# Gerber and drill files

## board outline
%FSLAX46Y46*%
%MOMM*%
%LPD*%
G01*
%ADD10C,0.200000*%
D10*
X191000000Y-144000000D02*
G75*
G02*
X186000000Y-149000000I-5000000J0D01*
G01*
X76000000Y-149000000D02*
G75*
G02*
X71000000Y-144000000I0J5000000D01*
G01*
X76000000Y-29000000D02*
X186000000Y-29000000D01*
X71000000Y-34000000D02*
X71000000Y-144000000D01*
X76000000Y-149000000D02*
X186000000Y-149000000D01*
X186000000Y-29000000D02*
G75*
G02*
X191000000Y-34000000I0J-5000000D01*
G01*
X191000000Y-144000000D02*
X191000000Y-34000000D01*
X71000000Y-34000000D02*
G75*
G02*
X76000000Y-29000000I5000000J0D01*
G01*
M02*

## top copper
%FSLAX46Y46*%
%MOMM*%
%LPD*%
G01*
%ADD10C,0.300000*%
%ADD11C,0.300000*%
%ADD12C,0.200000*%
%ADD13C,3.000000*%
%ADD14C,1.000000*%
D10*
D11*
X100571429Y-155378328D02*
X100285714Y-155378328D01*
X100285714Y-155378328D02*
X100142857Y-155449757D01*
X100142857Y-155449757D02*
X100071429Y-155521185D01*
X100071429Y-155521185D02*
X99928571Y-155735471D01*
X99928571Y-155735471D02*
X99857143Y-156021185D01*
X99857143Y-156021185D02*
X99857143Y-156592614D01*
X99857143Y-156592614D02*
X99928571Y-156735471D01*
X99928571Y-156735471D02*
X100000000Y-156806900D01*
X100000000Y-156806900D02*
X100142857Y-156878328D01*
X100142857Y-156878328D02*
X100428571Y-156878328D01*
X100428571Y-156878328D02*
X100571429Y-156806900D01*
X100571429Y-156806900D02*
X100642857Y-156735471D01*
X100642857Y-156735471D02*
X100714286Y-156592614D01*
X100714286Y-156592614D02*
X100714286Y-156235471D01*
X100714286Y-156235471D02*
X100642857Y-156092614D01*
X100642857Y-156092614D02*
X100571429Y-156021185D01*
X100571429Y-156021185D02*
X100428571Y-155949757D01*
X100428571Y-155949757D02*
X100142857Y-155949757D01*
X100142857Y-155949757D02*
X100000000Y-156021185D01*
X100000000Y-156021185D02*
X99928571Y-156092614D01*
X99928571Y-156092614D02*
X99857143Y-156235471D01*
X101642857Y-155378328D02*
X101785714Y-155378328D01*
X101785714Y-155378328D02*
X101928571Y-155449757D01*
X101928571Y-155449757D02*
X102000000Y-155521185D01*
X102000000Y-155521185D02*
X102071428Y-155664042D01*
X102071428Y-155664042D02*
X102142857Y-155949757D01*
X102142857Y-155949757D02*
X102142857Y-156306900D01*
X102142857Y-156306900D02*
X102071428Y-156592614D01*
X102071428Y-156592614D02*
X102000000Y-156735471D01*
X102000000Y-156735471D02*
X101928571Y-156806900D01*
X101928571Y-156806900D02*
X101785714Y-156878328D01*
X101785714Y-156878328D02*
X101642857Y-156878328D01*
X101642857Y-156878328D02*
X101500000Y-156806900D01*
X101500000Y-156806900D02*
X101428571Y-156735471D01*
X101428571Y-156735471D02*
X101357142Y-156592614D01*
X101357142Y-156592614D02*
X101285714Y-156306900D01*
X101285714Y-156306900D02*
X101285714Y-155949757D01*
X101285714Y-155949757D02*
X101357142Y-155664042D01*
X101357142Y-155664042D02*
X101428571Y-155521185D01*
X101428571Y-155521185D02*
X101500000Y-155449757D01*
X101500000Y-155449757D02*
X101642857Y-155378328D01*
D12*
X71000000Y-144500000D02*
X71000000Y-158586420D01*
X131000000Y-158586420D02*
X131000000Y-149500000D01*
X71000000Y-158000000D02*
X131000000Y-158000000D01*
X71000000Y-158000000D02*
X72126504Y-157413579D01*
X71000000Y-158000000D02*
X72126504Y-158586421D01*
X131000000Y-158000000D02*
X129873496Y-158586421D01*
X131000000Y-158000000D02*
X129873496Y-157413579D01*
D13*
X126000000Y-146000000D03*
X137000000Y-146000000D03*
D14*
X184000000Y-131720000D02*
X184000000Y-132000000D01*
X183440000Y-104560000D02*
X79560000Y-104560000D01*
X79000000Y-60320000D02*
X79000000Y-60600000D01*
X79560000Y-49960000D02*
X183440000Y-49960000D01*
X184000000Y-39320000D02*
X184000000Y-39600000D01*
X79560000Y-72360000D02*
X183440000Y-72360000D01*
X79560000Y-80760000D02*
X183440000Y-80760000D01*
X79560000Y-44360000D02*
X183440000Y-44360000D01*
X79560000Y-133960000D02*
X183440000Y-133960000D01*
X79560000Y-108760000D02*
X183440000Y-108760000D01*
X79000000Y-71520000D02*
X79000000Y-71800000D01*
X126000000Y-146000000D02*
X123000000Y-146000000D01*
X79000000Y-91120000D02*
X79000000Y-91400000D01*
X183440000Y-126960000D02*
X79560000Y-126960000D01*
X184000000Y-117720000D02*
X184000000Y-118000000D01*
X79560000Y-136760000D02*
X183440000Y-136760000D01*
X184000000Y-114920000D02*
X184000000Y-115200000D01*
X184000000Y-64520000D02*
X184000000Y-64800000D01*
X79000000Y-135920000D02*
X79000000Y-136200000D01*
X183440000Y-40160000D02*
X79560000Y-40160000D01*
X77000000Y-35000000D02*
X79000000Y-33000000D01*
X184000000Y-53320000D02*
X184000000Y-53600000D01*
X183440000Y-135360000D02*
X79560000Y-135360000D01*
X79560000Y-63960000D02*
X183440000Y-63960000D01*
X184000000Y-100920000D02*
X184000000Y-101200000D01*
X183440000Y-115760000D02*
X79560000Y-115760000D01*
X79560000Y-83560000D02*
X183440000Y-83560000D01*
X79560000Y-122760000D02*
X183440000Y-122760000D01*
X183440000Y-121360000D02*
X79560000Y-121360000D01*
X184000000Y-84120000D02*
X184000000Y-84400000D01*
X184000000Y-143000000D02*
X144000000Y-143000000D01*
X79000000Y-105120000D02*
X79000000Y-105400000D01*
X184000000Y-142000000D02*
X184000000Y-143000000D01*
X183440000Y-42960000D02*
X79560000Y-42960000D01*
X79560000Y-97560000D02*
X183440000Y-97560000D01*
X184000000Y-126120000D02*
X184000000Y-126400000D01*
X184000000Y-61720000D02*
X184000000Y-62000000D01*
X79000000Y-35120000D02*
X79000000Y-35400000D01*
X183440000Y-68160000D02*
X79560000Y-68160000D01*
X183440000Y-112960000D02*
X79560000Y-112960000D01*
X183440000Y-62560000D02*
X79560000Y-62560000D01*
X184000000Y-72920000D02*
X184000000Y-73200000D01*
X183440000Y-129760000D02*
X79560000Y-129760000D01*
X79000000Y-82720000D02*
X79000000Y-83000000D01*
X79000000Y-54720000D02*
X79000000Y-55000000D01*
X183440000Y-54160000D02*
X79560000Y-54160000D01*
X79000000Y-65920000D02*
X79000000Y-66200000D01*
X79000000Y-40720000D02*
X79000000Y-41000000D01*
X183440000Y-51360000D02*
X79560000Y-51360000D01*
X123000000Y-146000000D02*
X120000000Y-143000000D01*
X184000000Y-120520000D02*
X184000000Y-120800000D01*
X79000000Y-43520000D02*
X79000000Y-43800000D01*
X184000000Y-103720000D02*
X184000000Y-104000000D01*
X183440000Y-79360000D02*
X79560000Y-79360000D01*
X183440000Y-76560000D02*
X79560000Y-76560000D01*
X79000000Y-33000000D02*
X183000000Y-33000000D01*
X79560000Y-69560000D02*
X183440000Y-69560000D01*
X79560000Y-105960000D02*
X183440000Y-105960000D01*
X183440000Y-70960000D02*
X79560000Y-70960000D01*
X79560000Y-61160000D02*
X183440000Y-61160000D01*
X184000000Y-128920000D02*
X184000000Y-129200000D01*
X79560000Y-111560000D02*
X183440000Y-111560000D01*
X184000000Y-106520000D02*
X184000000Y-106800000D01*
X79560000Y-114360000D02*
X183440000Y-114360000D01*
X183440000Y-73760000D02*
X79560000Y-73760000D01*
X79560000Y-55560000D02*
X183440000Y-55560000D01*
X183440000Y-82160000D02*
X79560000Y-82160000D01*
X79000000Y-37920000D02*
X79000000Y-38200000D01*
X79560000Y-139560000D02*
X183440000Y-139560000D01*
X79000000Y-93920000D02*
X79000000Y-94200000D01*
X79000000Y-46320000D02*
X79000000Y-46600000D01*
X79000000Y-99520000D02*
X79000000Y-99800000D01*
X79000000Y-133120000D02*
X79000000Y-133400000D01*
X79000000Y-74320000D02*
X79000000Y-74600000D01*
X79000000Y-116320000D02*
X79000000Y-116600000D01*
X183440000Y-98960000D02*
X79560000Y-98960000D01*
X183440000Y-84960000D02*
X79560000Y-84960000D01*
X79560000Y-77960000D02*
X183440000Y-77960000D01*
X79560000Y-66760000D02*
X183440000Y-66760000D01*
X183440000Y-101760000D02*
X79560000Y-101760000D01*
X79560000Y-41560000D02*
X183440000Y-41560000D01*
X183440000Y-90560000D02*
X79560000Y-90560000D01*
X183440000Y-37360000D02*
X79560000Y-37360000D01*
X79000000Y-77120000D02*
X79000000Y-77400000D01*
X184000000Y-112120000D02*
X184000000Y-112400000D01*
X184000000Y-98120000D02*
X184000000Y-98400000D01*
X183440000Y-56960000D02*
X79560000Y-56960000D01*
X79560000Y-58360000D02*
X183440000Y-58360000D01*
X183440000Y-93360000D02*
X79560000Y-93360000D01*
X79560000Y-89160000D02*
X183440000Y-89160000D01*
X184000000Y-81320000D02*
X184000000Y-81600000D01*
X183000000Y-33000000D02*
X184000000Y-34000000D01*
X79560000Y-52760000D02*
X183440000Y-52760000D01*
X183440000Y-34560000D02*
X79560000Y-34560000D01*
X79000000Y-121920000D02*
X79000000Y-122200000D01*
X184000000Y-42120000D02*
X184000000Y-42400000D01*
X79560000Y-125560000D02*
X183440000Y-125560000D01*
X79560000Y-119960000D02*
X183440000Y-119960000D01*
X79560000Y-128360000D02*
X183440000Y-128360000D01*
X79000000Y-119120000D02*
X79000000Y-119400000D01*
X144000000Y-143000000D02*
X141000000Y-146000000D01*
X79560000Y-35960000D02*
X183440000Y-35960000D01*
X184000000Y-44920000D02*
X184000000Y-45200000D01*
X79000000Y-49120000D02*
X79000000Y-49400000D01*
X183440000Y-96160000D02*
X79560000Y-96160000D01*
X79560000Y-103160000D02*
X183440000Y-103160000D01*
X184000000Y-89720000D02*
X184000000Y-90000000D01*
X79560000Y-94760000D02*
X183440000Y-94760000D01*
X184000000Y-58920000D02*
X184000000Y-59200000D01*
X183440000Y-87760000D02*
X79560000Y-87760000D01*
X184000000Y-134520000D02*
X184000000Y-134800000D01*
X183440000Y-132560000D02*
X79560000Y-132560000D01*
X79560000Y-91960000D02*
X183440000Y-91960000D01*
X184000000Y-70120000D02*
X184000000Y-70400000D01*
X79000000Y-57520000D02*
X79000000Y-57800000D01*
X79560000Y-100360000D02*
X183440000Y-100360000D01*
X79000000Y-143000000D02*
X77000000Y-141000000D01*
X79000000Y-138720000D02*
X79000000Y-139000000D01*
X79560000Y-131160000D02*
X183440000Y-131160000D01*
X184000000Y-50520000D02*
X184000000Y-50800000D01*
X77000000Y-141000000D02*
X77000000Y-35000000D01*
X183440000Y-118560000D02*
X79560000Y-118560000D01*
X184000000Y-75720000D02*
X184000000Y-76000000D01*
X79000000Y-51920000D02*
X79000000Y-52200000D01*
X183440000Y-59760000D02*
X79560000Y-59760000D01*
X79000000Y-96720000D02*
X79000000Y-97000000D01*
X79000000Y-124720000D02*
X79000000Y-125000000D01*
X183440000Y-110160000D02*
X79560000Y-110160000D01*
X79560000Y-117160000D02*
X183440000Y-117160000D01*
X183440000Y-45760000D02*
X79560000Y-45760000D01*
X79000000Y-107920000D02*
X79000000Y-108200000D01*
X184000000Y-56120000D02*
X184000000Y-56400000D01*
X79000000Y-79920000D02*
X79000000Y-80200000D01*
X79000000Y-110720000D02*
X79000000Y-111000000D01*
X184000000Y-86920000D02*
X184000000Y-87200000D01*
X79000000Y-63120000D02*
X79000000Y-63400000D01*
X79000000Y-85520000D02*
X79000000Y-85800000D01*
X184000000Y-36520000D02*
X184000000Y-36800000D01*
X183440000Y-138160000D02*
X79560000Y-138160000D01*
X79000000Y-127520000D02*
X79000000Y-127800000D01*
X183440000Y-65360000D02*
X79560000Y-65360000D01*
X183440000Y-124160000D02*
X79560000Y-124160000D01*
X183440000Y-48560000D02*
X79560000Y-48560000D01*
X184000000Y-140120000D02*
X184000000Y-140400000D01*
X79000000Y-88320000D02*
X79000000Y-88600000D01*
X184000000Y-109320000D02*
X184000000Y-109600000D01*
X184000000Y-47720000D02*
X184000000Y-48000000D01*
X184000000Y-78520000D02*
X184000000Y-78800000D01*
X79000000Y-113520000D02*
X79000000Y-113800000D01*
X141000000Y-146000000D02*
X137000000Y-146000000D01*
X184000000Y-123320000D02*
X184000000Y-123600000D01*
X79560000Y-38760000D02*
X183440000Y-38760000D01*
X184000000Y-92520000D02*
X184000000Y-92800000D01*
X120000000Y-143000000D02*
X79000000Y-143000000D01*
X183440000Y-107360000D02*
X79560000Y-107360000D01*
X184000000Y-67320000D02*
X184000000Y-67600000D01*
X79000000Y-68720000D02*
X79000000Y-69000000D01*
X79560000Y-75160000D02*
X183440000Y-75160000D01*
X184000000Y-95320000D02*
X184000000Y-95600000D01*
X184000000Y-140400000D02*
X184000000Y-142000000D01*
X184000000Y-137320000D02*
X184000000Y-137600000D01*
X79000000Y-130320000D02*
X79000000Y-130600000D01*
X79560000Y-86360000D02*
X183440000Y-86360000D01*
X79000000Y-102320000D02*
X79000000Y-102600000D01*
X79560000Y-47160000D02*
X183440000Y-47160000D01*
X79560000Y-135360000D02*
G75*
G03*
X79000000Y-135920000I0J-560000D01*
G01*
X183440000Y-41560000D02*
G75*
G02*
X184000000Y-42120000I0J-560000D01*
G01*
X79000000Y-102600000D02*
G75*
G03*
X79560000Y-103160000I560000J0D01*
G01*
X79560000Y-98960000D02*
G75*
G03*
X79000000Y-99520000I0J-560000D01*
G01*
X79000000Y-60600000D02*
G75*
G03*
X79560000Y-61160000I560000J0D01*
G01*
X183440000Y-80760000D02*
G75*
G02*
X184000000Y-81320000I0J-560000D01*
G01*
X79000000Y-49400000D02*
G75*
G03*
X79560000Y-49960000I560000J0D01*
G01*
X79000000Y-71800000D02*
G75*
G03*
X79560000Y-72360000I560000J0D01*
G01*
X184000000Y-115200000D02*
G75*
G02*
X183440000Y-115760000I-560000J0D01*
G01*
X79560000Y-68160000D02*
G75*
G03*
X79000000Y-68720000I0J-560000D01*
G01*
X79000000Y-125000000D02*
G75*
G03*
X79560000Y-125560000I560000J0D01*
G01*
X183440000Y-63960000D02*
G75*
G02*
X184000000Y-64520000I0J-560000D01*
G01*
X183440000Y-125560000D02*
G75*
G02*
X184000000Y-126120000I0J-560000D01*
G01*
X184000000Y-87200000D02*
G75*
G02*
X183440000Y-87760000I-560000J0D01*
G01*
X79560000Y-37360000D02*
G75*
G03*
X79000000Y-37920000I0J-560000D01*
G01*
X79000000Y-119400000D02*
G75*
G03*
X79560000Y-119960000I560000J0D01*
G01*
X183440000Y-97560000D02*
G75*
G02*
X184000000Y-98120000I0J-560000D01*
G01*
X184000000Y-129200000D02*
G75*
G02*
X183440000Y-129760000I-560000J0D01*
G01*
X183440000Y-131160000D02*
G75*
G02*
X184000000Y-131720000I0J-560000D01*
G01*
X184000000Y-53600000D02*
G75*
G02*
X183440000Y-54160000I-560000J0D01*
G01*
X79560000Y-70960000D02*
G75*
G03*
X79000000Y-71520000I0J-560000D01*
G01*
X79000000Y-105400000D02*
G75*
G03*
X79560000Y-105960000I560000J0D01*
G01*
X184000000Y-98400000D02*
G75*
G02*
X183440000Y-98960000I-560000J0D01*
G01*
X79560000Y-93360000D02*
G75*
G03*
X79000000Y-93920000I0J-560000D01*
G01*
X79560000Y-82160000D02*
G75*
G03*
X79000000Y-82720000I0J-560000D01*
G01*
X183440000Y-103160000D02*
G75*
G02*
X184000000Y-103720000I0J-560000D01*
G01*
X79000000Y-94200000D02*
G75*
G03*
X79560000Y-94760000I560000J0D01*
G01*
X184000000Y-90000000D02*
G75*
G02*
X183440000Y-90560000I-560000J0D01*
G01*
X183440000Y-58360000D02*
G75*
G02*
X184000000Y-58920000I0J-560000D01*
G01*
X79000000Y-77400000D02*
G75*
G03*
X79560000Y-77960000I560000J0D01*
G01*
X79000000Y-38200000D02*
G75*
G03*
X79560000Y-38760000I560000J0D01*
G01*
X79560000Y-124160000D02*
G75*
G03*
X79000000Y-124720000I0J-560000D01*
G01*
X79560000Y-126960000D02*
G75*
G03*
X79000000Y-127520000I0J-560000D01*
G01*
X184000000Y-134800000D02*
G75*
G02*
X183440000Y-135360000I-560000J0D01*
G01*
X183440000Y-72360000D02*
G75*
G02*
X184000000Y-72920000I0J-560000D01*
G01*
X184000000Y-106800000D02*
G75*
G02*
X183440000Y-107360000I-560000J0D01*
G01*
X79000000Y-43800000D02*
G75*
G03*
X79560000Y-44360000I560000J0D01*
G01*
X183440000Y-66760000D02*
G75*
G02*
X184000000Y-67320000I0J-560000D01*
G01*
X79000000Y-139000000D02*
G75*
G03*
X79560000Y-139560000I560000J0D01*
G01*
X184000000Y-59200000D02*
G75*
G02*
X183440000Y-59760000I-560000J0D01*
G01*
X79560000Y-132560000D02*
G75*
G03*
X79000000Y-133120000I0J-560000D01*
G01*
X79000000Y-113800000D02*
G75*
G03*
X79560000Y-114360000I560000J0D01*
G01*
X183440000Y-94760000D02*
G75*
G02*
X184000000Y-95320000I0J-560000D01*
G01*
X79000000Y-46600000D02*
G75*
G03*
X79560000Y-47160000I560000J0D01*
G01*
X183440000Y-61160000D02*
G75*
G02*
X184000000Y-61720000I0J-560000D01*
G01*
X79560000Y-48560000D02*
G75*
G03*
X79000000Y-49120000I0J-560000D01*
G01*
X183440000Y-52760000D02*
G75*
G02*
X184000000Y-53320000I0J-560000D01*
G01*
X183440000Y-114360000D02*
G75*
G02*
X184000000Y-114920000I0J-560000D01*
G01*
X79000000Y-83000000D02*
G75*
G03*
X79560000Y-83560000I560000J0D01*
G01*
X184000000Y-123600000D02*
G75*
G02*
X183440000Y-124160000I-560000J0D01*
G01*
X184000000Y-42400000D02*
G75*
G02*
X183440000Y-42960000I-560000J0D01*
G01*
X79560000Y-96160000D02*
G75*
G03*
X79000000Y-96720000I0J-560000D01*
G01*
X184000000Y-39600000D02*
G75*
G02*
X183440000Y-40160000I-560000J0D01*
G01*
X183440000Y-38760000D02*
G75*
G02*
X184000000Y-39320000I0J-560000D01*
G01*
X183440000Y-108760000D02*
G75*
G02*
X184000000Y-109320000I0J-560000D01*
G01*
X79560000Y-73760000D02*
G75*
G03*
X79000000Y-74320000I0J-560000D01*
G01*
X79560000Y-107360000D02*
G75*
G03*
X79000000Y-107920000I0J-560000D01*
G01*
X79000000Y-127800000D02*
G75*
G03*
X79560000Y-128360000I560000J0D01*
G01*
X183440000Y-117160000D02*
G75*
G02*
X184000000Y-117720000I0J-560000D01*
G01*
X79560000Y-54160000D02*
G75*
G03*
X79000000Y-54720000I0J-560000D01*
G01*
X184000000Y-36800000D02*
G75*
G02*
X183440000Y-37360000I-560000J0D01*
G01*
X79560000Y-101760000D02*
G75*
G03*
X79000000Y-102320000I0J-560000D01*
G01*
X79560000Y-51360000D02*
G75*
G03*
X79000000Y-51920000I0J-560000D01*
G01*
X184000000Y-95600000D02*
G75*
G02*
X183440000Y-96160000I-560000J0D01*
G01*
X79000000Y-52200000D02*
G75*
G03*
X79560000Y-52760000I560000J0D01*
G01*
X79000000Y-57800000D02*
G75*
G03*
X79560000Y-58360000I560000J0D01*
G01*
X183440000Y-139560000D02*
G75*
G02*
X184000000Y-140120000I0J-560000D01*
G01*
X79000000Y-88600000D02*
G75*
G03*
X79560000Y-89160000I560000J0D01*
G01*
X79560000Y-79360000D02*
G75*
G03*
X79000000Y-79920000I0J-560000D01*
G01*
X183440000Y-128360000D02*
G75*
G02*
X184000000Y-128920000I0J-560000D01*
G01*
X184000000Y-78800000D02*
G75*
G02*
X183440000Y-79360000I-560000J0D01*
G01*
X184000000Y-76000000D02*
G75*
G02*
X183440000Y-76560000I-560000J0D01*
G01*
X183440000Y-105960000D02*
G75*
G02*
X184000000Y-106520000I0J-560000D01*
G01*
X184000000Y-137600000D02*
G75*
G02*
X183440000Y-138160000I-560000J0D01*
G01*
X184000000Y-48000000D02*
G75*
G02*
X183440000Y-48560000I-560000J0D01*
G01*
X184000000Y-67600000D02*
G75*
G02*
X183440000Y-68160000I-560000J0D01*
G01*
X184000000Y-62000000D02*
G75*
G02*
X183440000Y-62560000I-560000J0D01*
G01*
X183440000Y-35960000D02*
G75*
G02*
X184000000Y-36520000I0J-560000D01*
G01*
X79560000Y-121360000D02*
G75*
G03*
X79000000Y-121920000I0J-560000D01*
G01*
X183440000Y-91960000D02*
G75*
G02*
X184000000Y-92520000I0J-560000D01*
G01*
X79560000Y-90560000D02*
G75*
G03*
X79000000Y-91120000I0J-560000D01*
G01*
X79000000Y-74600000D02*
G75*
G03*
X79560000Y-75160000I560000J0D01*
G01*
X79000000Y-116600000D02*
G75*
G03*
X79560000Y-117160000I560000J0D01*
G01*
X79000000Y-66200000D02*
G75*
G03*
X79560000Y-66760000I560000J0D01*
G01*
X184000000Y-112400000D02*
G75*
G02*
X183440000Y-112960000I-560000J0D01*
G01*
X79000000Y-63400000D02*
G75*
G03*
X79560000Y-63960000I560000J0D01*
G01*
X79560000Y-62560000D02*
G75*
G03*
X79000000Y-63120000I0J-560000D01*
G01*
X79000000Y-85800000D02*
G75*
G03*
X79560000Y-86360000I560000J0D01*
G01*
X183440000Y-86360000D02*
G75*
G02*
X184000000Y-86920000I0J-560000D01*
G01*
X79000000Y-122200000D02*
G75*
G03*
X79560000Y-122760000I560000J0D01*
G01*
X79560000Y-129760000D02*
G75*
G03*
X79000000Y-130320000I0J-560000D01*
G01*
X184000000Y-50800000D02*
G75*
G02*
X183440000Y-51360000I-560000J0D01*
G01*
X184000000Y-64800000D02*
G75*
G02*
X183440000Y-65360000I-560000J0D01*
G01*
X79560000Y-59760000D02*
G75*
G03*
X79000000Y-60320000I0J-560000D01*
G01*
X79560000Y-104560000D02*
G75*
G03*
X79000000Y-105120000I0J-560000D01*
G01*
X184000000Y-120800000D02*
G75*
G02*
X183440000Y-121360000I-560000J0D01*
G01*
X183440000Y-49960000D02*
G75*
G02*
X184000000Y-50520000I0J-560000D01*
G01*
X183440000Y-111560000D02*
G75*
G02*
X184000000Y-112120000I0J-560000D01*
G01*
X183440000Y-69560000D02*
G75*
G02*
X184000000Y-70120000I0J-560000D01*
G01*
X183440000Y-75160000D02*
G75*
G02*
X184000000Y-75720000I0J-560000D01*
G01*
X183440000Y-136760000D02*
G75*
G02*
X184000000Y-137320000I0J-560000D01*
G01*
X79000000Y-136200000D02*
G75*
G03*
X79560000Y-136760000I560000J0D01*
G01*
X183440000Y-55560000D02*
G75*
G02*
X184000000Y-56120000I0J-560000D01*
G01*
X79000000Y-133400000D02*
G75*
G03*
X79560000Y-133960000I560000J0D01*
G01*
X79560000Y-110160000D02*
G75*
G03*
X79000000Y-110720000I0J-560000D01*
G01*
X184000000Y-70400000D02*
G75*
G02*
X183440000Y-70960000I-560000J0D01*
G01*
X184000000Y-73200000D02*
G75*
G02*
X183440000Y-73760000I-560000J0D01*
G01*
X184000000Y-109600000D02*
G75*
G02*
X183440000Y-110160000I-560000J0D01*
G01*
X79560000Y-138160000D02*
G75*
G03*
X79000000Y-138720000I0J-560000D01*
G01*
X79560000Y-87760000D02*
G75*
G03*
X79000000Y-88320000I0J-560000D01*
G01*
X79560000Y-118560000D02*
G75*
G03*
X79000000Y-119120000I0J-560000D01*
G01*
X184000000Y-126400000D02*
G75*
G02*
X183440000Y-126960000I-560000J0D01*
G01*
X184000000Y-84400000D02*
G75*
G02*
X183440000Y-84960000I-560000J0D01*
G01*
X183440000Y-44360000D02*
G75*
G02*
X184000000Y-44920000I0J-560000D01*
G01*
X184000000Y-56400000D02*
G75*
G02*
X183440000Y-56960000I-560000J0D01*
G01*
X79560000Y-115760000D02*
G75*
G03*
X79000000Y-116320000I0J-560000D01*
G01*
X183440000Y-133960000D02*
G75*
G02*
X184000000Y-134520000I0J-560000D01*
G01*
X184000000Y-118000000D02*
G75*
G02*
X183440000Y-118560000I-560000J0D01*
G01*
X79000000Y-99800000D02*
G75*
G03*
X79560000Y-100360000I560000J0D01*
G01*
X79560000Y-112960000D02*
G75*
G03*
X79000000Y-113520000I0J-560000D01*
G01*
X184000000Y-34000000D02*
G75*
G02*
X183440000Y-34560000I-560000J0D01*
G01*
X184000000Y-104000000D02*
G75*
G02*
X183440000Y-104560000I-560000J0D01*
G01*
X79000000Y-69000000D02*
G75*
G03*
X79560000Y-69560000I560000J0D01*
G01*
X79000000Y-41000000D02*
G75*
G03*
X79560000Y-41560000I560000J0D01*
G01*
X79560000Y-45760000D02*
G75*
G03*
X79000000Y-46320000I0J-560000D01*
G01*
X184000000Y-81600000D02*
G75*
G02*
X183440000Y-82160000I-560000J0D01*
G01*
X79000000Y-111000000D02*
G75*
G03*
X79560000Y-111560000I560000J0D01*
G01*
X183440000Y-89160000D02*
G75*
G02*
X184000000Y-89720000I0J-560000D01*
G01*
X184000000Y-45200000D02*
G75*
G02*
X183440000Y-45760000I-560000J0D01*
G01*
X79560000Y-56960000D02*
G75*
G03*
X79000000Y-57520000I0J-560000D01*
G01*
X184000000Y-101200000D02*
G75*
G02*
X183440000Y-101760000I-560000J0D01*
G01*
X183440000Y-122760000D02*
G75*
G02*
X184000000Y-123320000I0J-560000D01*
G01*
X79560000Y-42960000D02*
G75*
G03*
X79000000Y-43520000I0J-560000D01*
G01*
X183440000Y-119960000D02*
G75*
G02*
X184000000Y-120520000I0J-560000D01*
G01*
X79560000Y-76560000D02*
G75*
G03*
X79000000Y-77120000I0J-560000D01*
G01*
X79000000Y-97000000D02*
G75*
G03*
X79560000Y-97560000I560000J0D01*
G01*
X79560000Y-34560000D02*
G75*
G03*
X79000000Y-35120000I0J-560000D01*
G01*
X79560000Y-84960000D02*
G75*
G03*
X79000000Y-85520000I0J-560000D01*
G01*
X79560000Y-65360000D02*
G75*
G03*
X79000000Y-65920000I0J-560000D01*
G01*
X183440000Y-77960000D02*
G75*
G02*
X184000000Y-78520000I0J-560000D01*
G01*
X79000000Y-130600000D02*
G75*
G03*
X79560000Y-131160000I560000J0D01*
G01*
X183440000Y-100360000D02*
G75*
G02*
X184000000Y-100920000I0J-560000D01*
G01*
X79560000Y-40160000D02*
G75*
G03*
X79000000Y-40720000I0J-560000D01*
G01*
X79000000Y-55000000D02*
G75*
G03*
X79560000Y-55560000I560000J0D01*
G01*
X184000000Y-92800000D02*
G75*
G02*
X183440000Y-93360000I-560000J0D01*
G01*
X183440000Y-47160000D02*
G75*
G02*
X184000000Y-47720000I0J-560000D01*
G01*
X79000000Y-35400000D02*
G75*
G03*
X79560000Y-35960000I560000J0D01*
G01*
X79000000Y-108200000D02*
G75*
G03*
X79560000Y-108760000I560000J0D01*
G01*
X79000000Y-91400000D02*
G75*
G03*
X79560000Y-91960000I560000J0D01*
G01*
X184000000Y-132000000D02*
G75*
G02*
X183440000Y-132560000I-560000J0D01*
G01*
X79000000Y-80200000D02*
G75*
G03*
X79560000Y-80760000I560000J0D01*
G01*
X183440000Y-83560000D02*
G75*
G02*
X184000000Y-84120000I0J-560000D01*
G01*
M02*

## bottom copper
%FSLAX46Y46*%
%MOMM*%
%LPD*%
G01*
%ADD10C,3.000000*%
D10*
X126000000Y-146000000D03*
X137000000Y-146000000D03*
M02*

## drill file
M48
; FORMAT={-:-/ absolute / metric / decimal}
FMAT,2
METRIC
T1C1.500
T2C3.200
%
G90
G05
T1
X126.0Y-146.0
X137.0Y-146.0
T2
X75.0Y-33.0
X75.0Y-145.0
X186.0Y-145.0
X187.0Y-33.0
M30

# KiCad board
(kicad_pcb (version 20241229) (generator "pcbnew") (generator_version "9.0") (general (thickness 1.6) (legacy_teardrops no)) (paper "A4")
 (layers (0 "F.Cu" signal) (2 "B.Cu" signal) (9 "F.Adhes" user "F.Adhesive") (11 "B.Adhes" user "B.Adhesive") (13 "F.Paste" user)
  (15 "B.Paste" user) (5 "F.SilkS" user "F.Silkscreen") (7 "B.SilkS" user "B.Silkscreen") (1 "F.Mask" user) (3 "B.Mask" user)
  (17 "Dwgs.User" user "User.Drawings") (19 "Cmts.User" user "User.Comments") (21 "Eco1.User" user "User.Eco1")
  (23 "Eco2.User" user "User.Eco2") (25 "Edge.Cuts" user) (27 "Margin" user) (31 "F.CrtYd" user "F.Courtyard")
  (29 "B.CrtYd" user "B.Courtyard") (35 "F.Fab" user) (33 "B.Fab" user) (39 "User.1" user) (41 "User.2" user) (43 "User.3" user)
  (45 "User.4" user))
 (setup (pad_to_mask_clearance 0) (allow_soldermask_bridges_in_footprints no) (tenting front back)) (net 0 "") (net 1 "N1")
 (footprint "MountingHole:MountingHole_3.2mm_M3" (layer "F.Cu") (at 187 33)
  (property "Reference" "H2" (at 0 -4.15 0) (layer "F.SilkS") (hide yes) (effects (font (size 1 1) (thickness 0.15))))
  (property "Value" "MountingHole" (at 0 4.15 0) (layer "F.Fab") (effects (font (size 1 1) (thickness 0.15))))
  (pad "" np_thru_hole circle (at 0 0) (size 3.2 3.2) (drill 3.2) (layers "*.Cu" "*.Mask")))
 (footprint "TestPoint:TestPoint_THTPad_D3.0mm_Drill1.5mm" (layer "F.Cu") (at 126 146)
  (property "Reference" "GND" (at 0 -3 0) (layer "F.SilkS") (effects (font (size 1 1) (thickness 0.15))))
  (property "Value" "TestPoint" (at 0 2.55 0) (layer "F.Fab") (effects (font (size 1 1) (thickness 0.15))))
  (pad "1" thru_hole circle (at 0 0) (size 3 3) (drill 1.5) (layers "*.Cu" "*.Mask") (remove_unused_layers no) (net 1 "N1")))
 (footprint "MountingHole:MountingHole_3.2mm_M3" (layer "F.Cu") (at 75 33)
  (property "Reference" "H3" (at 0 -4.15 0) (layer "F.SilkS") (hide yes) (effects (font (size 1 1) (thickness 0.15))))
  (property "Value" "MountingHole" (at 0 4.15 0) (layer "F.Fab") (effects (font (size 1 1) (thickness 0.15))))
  (pad "" np_thru_hole circle (at 0 0) (size 3.2 3.2) (drill 3.2) (layers "*.Cu" "*.Mask")))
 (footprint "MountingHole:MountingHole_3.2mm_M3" (layer "F.Cu") (at 186 145)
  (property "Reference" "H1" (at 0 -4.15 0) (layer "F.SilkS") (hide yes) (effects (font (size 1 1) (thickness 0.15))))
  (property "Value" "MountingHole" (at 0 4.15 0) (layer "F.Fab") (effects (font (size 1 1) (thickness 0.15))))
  (pad "" np_thru_hole circle (at 0 0) (size 3.2 3.2) (drill 3.2) (layers "*.Cu" "*.Mask")))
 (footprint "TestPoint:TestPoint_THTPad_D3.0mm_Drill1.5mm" (layer "F.Cu") (at 137 146)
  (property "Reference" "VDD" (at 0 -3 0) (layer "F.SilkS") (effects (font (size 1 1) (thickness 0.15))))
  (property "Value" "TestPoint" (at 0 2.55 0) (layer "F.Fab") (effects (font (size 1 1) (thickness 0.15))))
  (pad "1" thru_hole circle (at 0 0) (size 3 3) (drill 1.5) (layers "*.Cu" "*.Mask") (remove_unused_layers no) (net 1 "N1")))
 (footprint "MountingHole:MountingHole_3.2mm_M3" (layer "F.Cu") (at 75 145)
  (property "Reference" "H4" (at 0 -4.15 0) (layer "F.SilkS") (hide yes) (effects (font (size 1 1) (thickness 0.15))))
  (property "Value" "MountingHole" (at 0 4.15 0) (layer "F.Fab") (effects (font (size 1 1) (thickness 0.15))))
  (pad "" np_thru_hole circle (at 0 0) (size 3.2 3.2) (drill 3.2) (layers "*.Cu" "*.Mask")))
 (gr_arc (start 191 144) (mid 189.535534 147.535534) (end 186 149) (stroke (width 0.2) (type solid)) (layer "Edge.Cuts"))
 (gr_arc (start 76 149) (mid 72.464466 147.535534) (end 71 144) (stroke (width 0.2) (type solid)) (layer "Edge.Cuts"))
 (gr_line (start 76 29) (end 186 29) (stroke (width 0.2) (type solid)) (layer "Edge.Cuts"))
 (gr_line (start 71 34) (end 71 144) (stroke (width 0.2) (type solid)) (layer "Edge.Cuts"))
 (gr_line (start 76 149) (end 186 149) (stroke (width 0.2) (type solid)) (layer "Edge.Cuts"))
 (gr_arc (start 186 29) (mid 189.535534 30.464466) (end 191 34) (stroke (width 0.2) (type solid)) (layer "Edge.Cuts"))
 (gr_line (start 191 144) (end 191 34) (stroke (width 0.2) (type solid)) (layer "Edge.Cuts"))
 (gr_arc (start 71 34) (mid 72.464466 30.464466) (end 76 29) (stroke (width 0.2) (type solid)) (layer "Edge.Cuts"))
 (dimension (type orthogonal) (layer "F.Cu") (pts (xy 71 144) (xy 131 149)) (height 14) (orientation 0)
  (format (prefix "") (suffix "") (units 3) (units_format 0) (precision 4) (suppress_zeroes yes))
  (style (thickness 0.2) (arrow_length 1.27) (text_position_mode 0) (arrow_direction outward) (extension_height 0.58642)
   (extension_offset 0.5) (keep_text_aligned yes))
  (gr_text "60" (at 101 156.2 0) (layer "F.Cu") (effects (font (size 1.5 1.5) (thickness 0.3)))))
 (segment (start 184 131.72) (end 184 132) (width 1) (layer "F.Cu") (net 1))
 (segment (start 183.44 104.56) (end 79.56 104.56) (width 1) (layer "F.Cu") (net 1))
 (segment (start 79 60.32) (end 79 60.6) (width 1) (layer "F.Cu") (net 1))
 (segment (start 79.56 49.96) (end 183.44 49.96) (width 1) (layer "F.Cu") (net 1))
 (segment (start 184 39.32) (end 184 39.6) (width 1) (layer "F.Cu") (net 1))
 (segment (start 79.56 72.36) (end 183.44 72.36) (width 1) (layer "F.Cu") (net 1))
 (segment (start 79.56 80.76) (end 183.44 80.76) (width 1) (layer "F.Cu") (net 1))
 (segment (start 79.56 44.36) (end 183.44 44.36) (width 1) (layer "F.Cu") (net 1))
 (segment (start 79.56 133.96) (end 183.44 133.96) (width 1) (layer "F.Cu") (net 1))
 (segment (start 79.56 108.76) (end 183.44 108.76) (width 1) (layer "F.Cu") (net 1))
 (segment (start 79 71.52) (end 79 71.8) (width 1) (layer "F.Cu") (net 1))
 (segment (start 126 146) (end 123 146) (width 1) (layer "F.Cu") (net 1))
 (segment (start 79 91.12) (end 79 91.4) (width 1) (layer "F.Cu") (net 1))
 (segment (start 183.44 126.96) (end 79.56 126.96) (width 1) (layer "F.Cu") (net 1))
 (segment (start 184 117.72) (end 184 118) (width 1) (layer "F.Cu") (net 1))
 (segment (start 79.56 136.76) (end 183.44 136.76) (width 1) (layer "F.Cu") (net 1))
 (segment (start 184 114.92) (end 184 115.2) (width 1) (layer "F.Cu") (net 1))
 (segment (start 184 64.52) (end 184 64.8) (width 1) (layer "F.Cu") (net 1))
 (segment (start 79 135.92) (end 79 136.2) (width 1) (layer "F.Cu") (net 1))
 (segment (start 183.44 40.16) (end 79.56 40.16) (width 1) (layer "F.Cu") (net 1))
 (segment (start 77 35) (end 79 33) (width 1) (layer "F.Cu") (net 1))
 (segment (start 184 53.32) (end 184 53.6) (width 1) (layer "F.Cu") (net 1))
 (segment (start 183.44 135.36) (end 79.56 135.36) (width 1) (layer "F.Cu") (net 1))
 (segment (start 79.56 63.96) (end 183.44 63.96) (width 1) (layer "F.Cu") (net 1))
 (segment (start 184 100.92) (end 184 101.2) (width 1) (layer "F.Cu") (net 1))
 (segment (start 183.44 115.76) (end 79.56 115.76) (width 1) (layer "F.Cu") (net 1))
 (segment (start 79.56 83.56) (end 183.44 83.56) (width 1) (layer "F.Cu") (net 1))
 (segment (start 79.56 122.76) (end 183.44 122.76) (width 1) (layer "F.Cu") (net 1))
 (segment (start 183.44 121.36) (end 79.56 121.36) (width 1) (layer "F.Cu") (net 1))
 (segment (start 184 84.12) (end 184 84.4) (width 1) (layer "F.Cu") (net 1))
 (segment (start 184 143) (end 144 143) (width 1) (layer "F.Cu") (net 1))
 (segment (start 79 105.12) (end 79 105.4) (width 1) (layer "F.Cu") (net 1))
 (segment (start 184 142) (end 184 143) (width 1) (layer "F.Cu") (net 1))
 (segment (start 183.44 42.96) (end 79.56 42.96) (width 1) (layer "F.Cu") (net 1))
 (segment (start 79.56 97.56) (end 183.44 97.56) (width 1) (layer "F.Cu") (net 1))
 (segment (start 184 126.12) (end 184 126.4) (width 1) (layer "F.Cu") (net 1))
 (segment (start 184 61.72) (end 184 62) (width 1) (layer "F.Cu") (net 1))
 (segment (start 79 35.12) (end 79 35.4) (width 1) (layer "F.Cu") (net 1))
 (segment (start 183.44 68.16) (end 79.56 68.16) (width 1) (layer "F.Cu") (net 1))
 (segment (start 183.44 112.96) (end 79.56 112.96) (width 1) (layer "F.Cu") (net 1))
 (segment (start 183.44 62.56) (end 79.56 62.56) (width 1) (layer "F.Cu") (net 1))
 (segment (start 184 72.92) (end 184 73.2) (width 1) (layer "F.Cu") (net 1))
 (segment (start 183.44 129.76) (end 79.56 129.76) (width 1) (layer "F.Cu") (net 1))
 (segment (start 79 82.72) (end 79 83) (width 1) (layer "F.Cu") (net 1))
 (segment (start 79 54.72) (end 79 55) (width 1) (layer "F.Cu") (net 1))
 (segment (start 183.44 54.16) (end 79.56 54.16) (width 1) (layer "F.Cu") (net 1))
 (segment (start 79 65.92) (end 79 66.2) (width 1) (layer "F.Cu") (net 1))
 (segment (start 79 40.72) (end 79 41) (width 1) (layer "F.Cu") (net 1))
 (segment (start 183.44 51.36) (end 79.56 51.36) (width 1) (layer "F.Cu") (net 1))
 (segment (start 123 146) (end 120 143) (width 1) (layer "F.Cu") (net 1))
 (segment (start 184 120.52) (end 184 120.8) (width 1) (layer "F.Cu") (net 1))
 (segment (start 79 43.52) (end 79 43.8) (width 1) (layer "F.Cu") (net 1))
 (segment (start 184 103.72) (end 184 104) (width 1) (layer "F.Cu") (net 1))
 (segment (start 183.44 79.36) (end 79.56 79.36) (width 1) (layer "F.Cu") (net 1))
 (segment (start 183.44 76.56) (end 79.56 76.56) (width 1) (layer "F.Cu") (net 1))
 (segment (start 79 33) (end 183 33) (width 1) (layer "F.Cu") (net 1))
 (segment (start 79.56 69.56) (end 183.44 69.56) (width 1) (layer "F.Cu") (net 1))
 (segment (start 79.56 105.96) (end 183.44 105.96) (width 1) (layer "F.Cu") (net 1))
 (segment (start 183.44 70.96) (end 79.56 70.96) (width 1) (layer "F.Cu") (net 1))
 (segment (start 79.56 61.16) (end 183.44 61.16) (width 1) (layer "F.Cu") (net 1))
 (segment (start 184 128.92) (end 184 129.2) (width 1) (layer "F.Cu") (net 1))
 (segment (start 79.56 111.56) (end 183.44 111.56) (width 1) (layer "F.Cu") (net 1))
 (segment (start 184 106.52) (end 184 106.8) (width 1) (layer "F.Cu") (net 1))
 (segment (start 79.56 114.36) (end 183.44 114.36) (width 1) (layer "F.Cu") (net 1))
 (segment (start 183.44 73.76) (end 79.56 73.76) (width 1) (layer "F.Cu") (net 1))
 (segment (start 79.56 55.56) (end 183.44 55.56) (width 1) (layer "F.Cu") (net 1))
 (segment (start 183.44 82.16) (end 79.56 82.16) (width 1) (layer "F.Cu") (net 1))
 (segment (start 79 37.92) (end 79 38.2) (width 1) (layer "F.Cu") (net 1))
 (segment (start 79.56 139.56) (end 183.44 139.56) (width 1) (layer "F.Cu") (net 1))
 (segment (start 79 93.92) (end 79 94.2) (width 1) (layer "F.Cu") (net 1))
 (segment (start 79 46.32) (end 79 46.6) (width 1) (layer "F.Cu") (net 1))
 (segment (start 79 99.52) (end 79 99.8) (width 1) (layer "F.Cu") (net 1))
 (segment (start 79 133.12) (end 79 133.4) (width 1) (layer "F.Cu") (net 1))
 (segment (start 79 74.32) (end 79 74.6) (width 1) (layer "F.Cu") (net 1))
 (segment (start 79 116.32) (end 79 116.6) (width 1) (layer "F.Cu") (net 1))
 (segment (start 183.44 98.96) (end 79.56 98.96) (width 1) (layer "F.Cu") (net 1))
 (segment (start 183.44 84.96) (end 79.56 84.96) (width 1) (layer "F.Cu") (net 1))
 (segment (start 79.56 77.96) (end 183.44 77.96) (width 1) (layer "F.Cu") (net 1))
 (segment (start 79.56 66.76) (end 183.44 66.76) (width 1) (layer "F.Cu") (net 1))
 (segment (start 183.44 101.76) (end 79.56 101.76) (width 1) (layer "F.Cu") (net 1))
 (segment (start 79.56 41.56) (end 183.44 41.56) (width 1) (layer "F.Cu") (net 1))
 (segment (start 183.44 90.56) (end 79.56 90.56) (width 1) (layer "F.Cu") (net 1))
 (segment (start 183.44 37.36) (end 79.56 37.36) (width 1) (layer "F.Cu") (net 1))
 (segment (start 79 77.12) (end 79 77.4) (width 1) (layer "F.Cu") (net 1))
 (segment (start 184 112.12) (end 184 112.4) (width 1) (layer "F.Cu") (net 1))
 (segment (start 184 98.12) (end 184 98.4) (width 1) (layer "F.Cu") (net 1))
 (segment (start 183.44 56.96) (end 79.56 56.96) (width 1) (layer "F.Cu") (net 1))
 (segment (start 79.56 58.36) (end 183.44 58.36) (width 1) (layer "F.Cu") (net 1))
 (segment (start 183.44 93.36) (end 79.56 93.36) (width 1) (layer "F.Cu") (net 1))
 (segment (start 79.56 89.16) (end 183.44 89.16) (width 1) (layer "F.Cu") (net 1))
 (segment (start 184 81.32) (end 184 81.6) (width 1) (layer "F.Cu") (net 1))
 (segment (start 183 33) (end 184 34) (width 1) (layer "F.Cu") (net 1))
 (segment (start 79.56 52.76) (end 183.44 52.76) (width 1) (layer "F.Cu") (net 1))
 (segment (start 183.44 34.56) (end 79.56 34.56) (width 1) (layer "F.Cu") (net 1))
 (segment (start 79 121.92) (end 79 122.2) (width 1) (layer "F.Cu") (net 1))
 (segment (start 184 42.12) (end 184 42.4) (width 1) (layer "F.Cu") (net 1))
 (segment (start 79.56 125.56) (end 183.44 125.56) (width 1) (layer "F.Cu") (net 1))
 (segment (start 79.56 119.96) (end 183.44 119.96) (width 1) (layer "F.Cu") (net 1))
 (segment (start 79.56 128.36) (end 183.44 128.36) (width 1) (layer "F.Cu") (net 1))
 (segment (start 79 119.12) (end 79 119.4) (width 1) (layer "F.Cu") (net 1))
 (segment (start 144 143) (end 141 146) (width 1) (layer "F.Cu") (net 1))
 (segment (start 79.56 35.96) (end 183.44 35.96) (width 1) (layer "F.Cu") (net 1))
 (segment (start 184 44.92) (end 184 45.2) (width 1) (layer "F.Cu") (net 1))
 (segment (start 79 49.12) (end 79 49.4) (width 1) (layer "F.Cu") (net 1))
 (segment (start 183.44 96.16) (end 79.56 96.16) (width 1) (layer "F.Cu") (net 1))
 (segment (start 79.56 103.16) (end 183.44 103.16) (width 1) (layer "F.Cu") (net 1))
 (segment (start 184 89.72) (end 184 90) (width 1) (layer "F.Cu") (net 1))
 (segment (start 79.56 94.76) (end 183.44 94.76) (width 1) (layer "F.Cu") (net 1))
 (segment (start 184 58.92) (end 184 59.2) (width 1) (layer "F.Cu") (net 1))
 (segment (start 183.44 87.76) (end 79.56 87.76) (width 1) (layer "F.Cu") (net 1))
 (segment (start 184 134.52) (end 184 134.8) (width 1) (layer "F.Cu") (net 1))
 (segment (start 183.44 132.56) (end 79.56 132.56) (width 1) (layer "F.Cu") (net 1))
 (segment (start 79.56 91.96) (end 183.44 91.96) (width 1) (layer "F.Cu") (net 1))
 (segment (start 184 70.12) (end 184 70.4) (width 1) (layer "F.Cu") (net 1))
 (segment (start 79 57.52) (end 79 57.8) (width 1) (layer "F.Cu") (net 1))
 (segment (start 79.56 100.36) (end 183.44 100.36) (width 1) (layer "F.Cu") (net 1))
 (segment (start 79 143) (end 77 141) (width 1) (layer "F.Cu") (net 1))
 (segment (start 79 138.72) (end 79 139) (width 1) (layer "F.Cu") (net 1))
 (segment (start 79.56 131.16) (end 183.44 131.16) (width 1) (layer "F.Cu") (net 1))
 (segment (start 184 50.52) (end 184 50.8) (width 1) (layer "F.Cu") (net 1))
 (segment (start 77 141) (end 77 35) (width 1) (layer "F.Cu") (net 1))
 (segment (start 183.44 118.56) (end 79.56 118.56) (width 1) (layer "F.Cu") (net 1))
 (segment (start 184 75.72) (end 184 76) (width 1) (layer "F.Cu") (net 1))
 (segment (start 79 51.92) (end 79 52.2) (width 1) (layer "F.Cu") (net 1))
 (segment (start 183.44 59.76) (end 79.56 59.76) (width 1) (layer "F.Cu") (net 1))
 (segment (start 79 96.72) (end 79 97) (width 1) (layer "F.Cu") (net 1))
 (segment (start 79 124.72) (end 79 125) (width 1) (layer "F.Cu") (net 1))
 (segment (start 183.44 110.16) (end 79.56 110.16) (width 1) (layer "F.Cu") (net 1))
 (segment (start 79.56 117.16) (end 183.44 117.16) (width 1) (layer "F.Cu") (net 1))
 (segment (start 183.44 45.76) (end 79.56 45.76) (width 1) (layer "F.Cu") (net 1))
 (segment (start 79 107.92) (end 79 108.2) (width 1) (layer "F.Cu") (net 1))
 (segment (start 184 56.12) (end 184 56.4) (width 1) (layer "F.Cu") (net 1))
 (segment (start 79 79.92) (end 79 80.2) (width 1) (layer "F.Cu") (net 1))
 (segment (start 79 110.72) (end 79 111) (width 1) (layer "F.Cu") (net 1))
 (segment (start 184 86.92) (end 184 87.2) (width 1) (layer "F.Cu") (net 1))
 (segment (start 79 63.12) (end 79 63.4) (width 1) (layer "F.Cu") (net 1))
 (segment (start 79 85.52) (end 79 85.8) (width 1) (layer "F.Cu") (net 1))
 (segment (start 184 36.52) (end 184 36.8) (width 1) (layer "F.Cu") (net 1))
 (segment (start 183.44 138.16) (end 79.56 138.16) (width 1) (layer "F.Cu") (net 1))
 (segment (start 79 127.52) (end 79 127.8) (width 1) (layer "F.Cu") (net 1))
 (segment (start 183.44 65.36) (end 79.56 65.36) (width 1) (layer "F.Cu") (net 1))
 (segment (start 183.44 124.16) (end 79.56 124.16) (width 1) (layer "F.Cu") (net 1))
 (segment (start 183.44 48.56) (end 79.56 48.56) (width 1) (layer "F.Cu") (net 1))
 (segment (start 184 140.12) (end 184 140.4) (width 1) (layer "F.Cu") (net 1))
 (segment (start 79 88.32) (end 79 88.6) (width 1) (layer "F.Cu") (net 1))
 (segment (start 184 109.32) (end 184 109.6) (width 1) (layer "F.Cu") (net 1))
 (segment (start 184 47.72) (end 184 48) (width 1) (layer "F.Cu") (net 1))
 (segment (start 184 78.52) (end 184 78.8) (width 1) (layer "F.Cu") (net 1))
 (segment (start 79 113.52) (end 79 113.8) (width 1) (layer "F.Cu") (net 1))
 (segment (start 141 146) (end 137 146) (width 1) (layer "F.Cu") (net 1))
 (segment (start 184 123.32) (end 184 123.6) (width 1) (layer "F.Cu") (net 1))
 (segment (start 79.56 38.76) (end 183.44 38.76) (width 1) (layer "F.Cu") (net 1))
 (segment (start 184 92.52) (end 184 92.8) (width 1) (layer "F.Cu") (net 1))
 (segment (start 120 143) (end 79 143) (width 1) (layer "F.Cu") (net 1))
 (segment (start 183.44 107.36) (end 79.56 107.36) (width 1) (layer "F.Cu") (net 1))
 (segment (start 184 67.32) (end 184 67.6) (width 1) (layer "F.Cu") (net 1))
 (segment (start 79 68.72) (end 79 69) (width 1) (layer "F.Cu") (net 1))
 (segment (start 79.56 75.16) (end 183.44 75.16) (width 1) (layer "F.Cu") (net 1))
 (segment (start 184 95.32) (end 184 95.6) (width 1) (layer "F.Cu") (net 1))
 (segment (start 184 140.4) (end 184 142) (width 1) (layer "F.Cu") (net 1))
 (segment (start 184 137.32) (end 184 137.6) (width 1) (layer "F.Cu") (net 1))
 (segment (start 79 130.32) (end 79 130.6) (width 1) (layer "F.Cu") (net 1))
 (segment (start 79.56 86.36) (end 183.44 86.36) (width 1) (layer "F.Cu") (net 1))
 (segment (start 79 102.32) (end 79 102.6) (width 1) (layer "F.Cu") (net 1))
 (segment (start 79.56 47.16) (end 183.44 47.16) (width 1) (layer "F.Cu") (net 1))
 (arc (start 79.56 135.36) (mid 79.16402 135.52402) (end 79 135.92) (width 1) (layer "F.Cu") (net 1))
 (arc (start 183.44 41.56) (mid 183.83598 41.72402) (end 184 42.12) (width 1) (layer "F.Cu") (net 1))
 (arc (start 79 102.6) (mid 79.16402 102.99598) (end 79.56 103.16) (width 1) (layer "F.Cu") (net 1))
 (arc (start 79.56 98.96) (mid 79.16402 99.12402) (end 79 99.52) (width 1) (layer "F.Cu") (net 1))
 (arc (start 79 60.6) (mid 79.16402 60.99598) (end 79.56 61.16) (width 1) (layer "F.Cu") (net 1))
 (arc (start 183.44 80.76) (mid 183.83598 80.92402) (end 184 81.32) (width 1) (layer "F.Cu") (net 1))
 (arc (start 79 49.4) (mid 79.16402 49.79598) (end 79.56 49.96) (width 1) (layer "F.Cu") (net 1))
 (arc (start 79 71.8) (mid 79.16402 72.19598) (end 79.56 72.36) (width 1) (layer "F.Cu") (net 1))
 (arc (start 184 115.2) (mid 183.83598 115.59598) (end 183.44 115.76) (width 1) (layer "F.Cu") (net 1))
 (arc (start 79.56 68.16) (mid 79.16402 68.32402) (end 79 68.72) (width 1) (layer "F.Cu") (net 1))
 (arc (start 79 125) (mid 79.16402 125.39598) (end 79.56 125.56) (width 1) (layer "F.Cu") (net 1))
 (arc (start 183.44 63.96) (mid 183.83598 64.12402) (end 184 64.52) (width 1) (layer "F.Cu") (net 1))
 (arc (start 183.44 125.56) (mid 183.83598 125.72402) (end 184 126.12) (width 1) (layer "F.Cu") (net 1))
 (arc (start 184 87.2) (mid 183.83598 87.59598) (end 183.44 87.76) (width 1) (layer "F.Cu") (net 1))
 (arc (start 79.56 37.36) (mid 79.16402 37.52402) (end 79 37.92) (width 1) (layer "F.Cu") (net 1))
 (arc (start 79 119.4) (mid 79.16402 119.79598) (end 79.56 119.96) (width 1) (layer "F.Cu") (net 1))
 (arc (start 183.44 97.56) (mid 183.83598 97.72402) (end 184 98.12) (width 1) (layer "F.Cu") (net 1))
 (arc (start 184 129.2) (mid 183.83598 129.59598) (end 183.44 129.76) (width 1) (layer "F.Cu") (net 1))
 (arc (start 183.44 131.16) (mid 183.83598 131.32402) (end 184 131.72) (width 1) (layer "F.Cu") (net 1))
 (arc (start 184 53.6) (mid 183.83598 53.99598) (end 183.44 54.16) (width 1) (layer "F.Cu") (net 1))
 (arc (start 79.56 70.96) (mid 79.16402 71.12402) (end 79 71.52) (width 1) (layer "F.Cu") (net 1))
 (arc (start 79 105.4) (mid 79.16402 105.79598) (end 79.56 105.96) (width 1) (layer "F.Cu") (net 1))
 (arc (start 184 98.4) (mid 183.83598 98.79598) (end 183.44 98.96) (width 1) (layer "F.Cu") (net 1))
 (arc (start 79.56 93.36) (mid 79.16402 93.52402) (end 79 93.92) (width 1) (layer "F.Cu") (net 1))
 (arc (start 79.56 82.16) (mid 79.16402 82.32402) (end 79 82.72) (width 1) (layer "F.Cu") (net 1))
 (arc (start 183.44 103.16) (mid 183.83598 103.32402) (end 184 103.72) (width 1) (layer "F.Cu") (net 1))
 (arc (start 79 94.2) (mid 79.16402 94.59598) (end 79.56 94.76) (width 1) (layer "F.Cu") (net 1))
 (arc (start 184 90) (mid 183.83598 90.39598) (end 183.44 90.56) (width 1) (layer "F.Cu") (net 1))
 (arc (start 183.44 58.36) (mid 183.83598 58.52402) (end 184 58.92) (width 1) (layer "F.Cu") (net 1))
 (arc (start 79 77.4) (mid 79.16402 77.79598) (end 79.56 77.96) (width 1) (layer "F.Cu") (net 1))
 (arc (start 79 38.2) (mid 79.16402 38.59598) (end 79.56 38.76) (width 1) (layer "F.Cu") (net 1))
 (arc (start 79.56 124.16) (mid 79.16402 124.32402) (end 79 124.72) (width 1) (layer "F.Cu") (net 1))
 (arc (start 79.56 126.96) (mid 79.16402 127.12402) (end 79 127.52) (width 1) (layer "F.Cu") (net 1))
 (arc (start 184 134.8) (mid 183.83598 135.19598) (end 183.44 135.36) (width 1) (layer "F.Cu") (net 1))
 (arc (start 183.44 72.36) (mid 183.83598 72.52402) (end 184 72.92) (width 1) (layer "F.Cu") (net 1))
 (arc (start 184 106.8) (mid 183.83598 107.19598) (end 183.44 107.36) (width 1) (layer "F.Cu") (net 1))
 (arc (start 79 43.8) (mid 79.16402 44.19598) (end 79.56 44.36) (width 1) (layer "F.Cu") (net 1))
 (arc (start 183.44 66.76) (mid 183.83598 66.92402) (end 184 67.32) (width 1) (layer "F.Cu") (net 1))
 (arc (start 79 139) (mid 79.16402 139.39598) (end 79.56 139.56) (width 1) (layer "F.Cu") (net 1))
 (arc (start 184 59.2) (mid 183.83598 59.59598) (end 183.44 59.76) (width 1) (layer "F.Cu") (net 1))
 (arc (start 79.56 132.56) (mid 79.16402 132.72402) (end 79 133.12) (width 1) (layer "F.Cu") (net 1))
 (arc (start 79 113.8) (mid 79.16402 114.19598) (end 79.56 114.36) (width 1) (layer "F.Cu") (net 1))
 (arc (start 183.44 94.76) (mid 183.83598 94.92402) (end 184 95.32) (width 1) (layer "F.Cu") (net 1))
 (arc (start 79 46.6) (mid 79.16402 46.99598) (end 79.56 47.16) (width 1) (layer "F.Cu") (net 1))
 (arc (start 183.44 61.16) (mid 183.83598 61.32402) (end 184 61.72) (width 1) (layer "F.Cu") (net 1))
 (arc (start 79.56 48.56) (mid 79.16402 48.72402) (end 79 49.12) (width 1) (layer "F.Cu") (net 1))
 (arc (start 183.44 52.76) (mid 183.83598 52.92402) (end 184 53.32) (width 1) (layer "F.Cu") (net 1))
 (arc (start 183.44 114.36) (mid 183.83598 114.52402) (end 184 114.92) (width 1) (layer "F.Cu") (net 1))
 (arc (start 79 83) (mid 79.16402 83.39598) (end 79.56 83.56) (width 1) (layer "F.Cu") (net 1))
 (arc (start 184 123.6) (mid 183.83598 123.99598) (end 183.44 124.16) (width 1) (layer "F.Cu") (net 1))
 (arc (start 184 42.4) (mid 183.83598 42.79598) (end 183.44 42.96) (width 1) (layer "F.Cu") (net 1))
 (arc (start 79.56 96.16) (mid 79.16402 96.32402) (end 79 96.72) (width 1) (layer "F.Cu") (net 1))
 (arc (start 184 39.6) (mid 183.83598 39.99598) (end 183.44 40.16) (width 1) (layer "F.Cu") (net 1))
 (arc (start 183.44 38.76) (mid 183.83598 38.92402) (end 184 39.32) (width 1) (layer "F.Cu") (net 1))
 (arc (start 183.44 108.76) (mid 183.83598 108.92402) (end 184 109.32) (width 1) (layer "F.Cu") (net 1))
 (arc (start 79.56 73.76) (mid 79.16402 73.92402) (end 79 74.32) (width 1) (layer "F.Cu") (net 1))
 (arc (start 79.56 107.36) (mid 79.16402 107.52402) (end 79 107.92) (width 1) (layer "F.Cu") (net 1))
 (arc (start 79 127.8) (mid 79.16402 128.19598) (end 79.56 128.36) (width 1) (layer "F.Cu") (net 1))
 (arc (start 183.44 117.16) (mid 183.83598 117.32402) (end 184 117.72) (width 1) (layer "F.Cu") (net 1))
 (arc (start 79.56 54.16) (mid 79.16402 54.32402) (end 79 54.72) (width 1) (layer "F.Cu") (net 1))
 (arc (start 184 36.8) (mid 183.83598 37.19598) (end 183.44 37.36) (width 1) (layer "F.Cu") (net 1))
 (arc (start 79.56 101.76) (mid 79.16402 101.92402) (end 79 102.32) (width 1) (layer "F.Cu") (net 1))
 (arc (start 79.56 51.36) (mid 79.16402 51.52402) (end 79 51.92) (width 1) (layer "F.Cu") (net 1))
 (arc (start 184 95.6) (mid 183.83598 95.99598) (end 183.44 96.16) (width 1) (layer "F.Cu") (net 1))
 (arc (start 79 52.2) (mid 79.16402 52.59598) (end 79.56 52.76) (width 1) (layer "F.Cu") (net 1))
 (arc (start 79 57.8) (mid 79.16402 58.19598) (end 79.56 58.36) (width 1) (layer "F.Cu") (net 1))
 (arc (start 183.44 139.56) (mid 183.83598 139.72402) (end 184 140.12) (width 1) (layer "F.Cu") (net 1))
 (arc (start 79 88.6) (mid 79.16402 88.99598) (end 79.56 89.16) (width 1) (layer "F.Cu") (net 1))
 (arc (start 79.56 79.36) (mid 79.16402 79.52402) (end 79 79.92) (width 1) (layer "F.Cu") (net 1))
 (arc (start 183.44 128.36) (mid 183.83598 128.52402) (end 184 128.92) (width 1) (layer "F.Cu") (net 1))
 (arc (start 184 78.8) (mid 183.83598 79.19598) (end 183.44 79.36) (width 1) (layer "F.Cu") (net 1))
 (arc (start 184 76) (mid 183.83598 76.39598) (end 183.44 76.56) (width 1) (layer "F.Cu") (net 1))
 (arc (start 183.44 105.96) (mid 183.83598 106.12402) (end 184 106.52) (width 1) (layer "F.Cu") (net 1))
 (arc (start 184 137.6) (mid 183.83598 137.99598) (end 183.44 138.16) (width 1) (layer "F.Cu") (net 1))
 (arc (start 184 48) (mid 183.83598 48.39598) (end 183.44 48.56) (width 1) (layer "F.Cu") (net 1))
 (arc (start 184 67.6) (mid 183.83598 67.99598) (end 183.44 68.16) (width 1) (layer "F.Cu") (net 1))
 (arc (start 184 62) (mid 183.83598 62.39598) (end 183.44 62.56) (width 1) (layer "F.Cu") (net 1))
 (arc (start 183.44 35.96) (mid 183.83598 36.12402) (end 184 36.52) (width 1) (layer "F.Cu") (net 1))
 (arc (start 79.56 121.36) (mid 79.16402 121.52402) (end 79 121.92) (width 1) (layer "F.Cu") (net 1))
 (arc (start 183.44 91.96) (mid 183.83598 92.12402) (end 184 92.52) (width 1) (layer "F.Cu") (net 1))
 (arc (start 79.56 90.56) (mid 79.16402 90.72402) (end 79 91.12) (width 1) (layer "F.Cu") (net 1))
 (arc (start 79 74.6) (mid 79.16402 74.99598) (end 79.56 75.16) (width 1) (layer "F.Cu") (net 1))
 (arc (start 79 116.6) (mid 79.16402 116.99598) (end 79.56 117.16) (width 1) (layer "F.Cu") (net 1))
 (arc (start 79 66.2) (mid 79.16402 66.59598) (end 79.56 66.76) (width 1) (layer "F.Cu") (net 1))
 (arc (start 184 112.4) (mid 183.83598 112.79598) (end 183.44 112.96) (width 1) (layer "F.Cu") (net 1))
 (arc (start 79 63.4) (mid 79.16402 63.79598) (end 79.56 63.96) (width 1) (layer "F.Cu") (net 1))
 (arc (start 79.56 62.56) (mid 79.16402 62.72402) (end 79 63.12) (width 1) (layer "F.Cu") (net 1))
 (arc (start 79 85.8) (mid 79.16402 86.19598) (end 79.56 86.36) (width 1) (layer "F.Cu") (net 1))
 (arc (start 183.44 86.36) (mid 183.83598 86.52402) (end 184 86.92) (width 1) (layer "F.Cu") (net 1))
 (arc (start 79 122.2) (mid 79.16402 122.59598) (end 79.56 122.76) (width 1) (layer "F.Cu") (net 1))
 (arc (start 79.56 129.76) (mid 79.16402 129.92402) (end 79 130.32) (width 1) (layer "F.Cu") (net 1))
 (arc (start 184 50.8) (mid 183.83598 51.19598) (end 183.44 51.36) (width 1) (layer "F.Cu") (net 1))
 (arc (start 184 64.8) (mid 183.83598 65.19598) (end 183.44 65.36) (width 1) (layer "F.Cu") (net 1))
 (arc (start 79.56 59.76) (mid 79.16402 59.92402) (end 79 60.32) (width 1) (layer "F.Cu") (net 1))
 (arc (start 79.56 104.56) (mid 79.16402 104.72402) (end 79 105.12) (width 1) (layer "F.Cu") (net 1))
 (arc (start 184 120.8) (mid 183.83598 121.19598) (end 183.44 121.36) (width 1) (layer "F.Cu") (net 1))
 (arc (start 183.44 49.96) (mid 183.83598 50.12402) (end 184 50.52) (width 1) (layer "F.Cu") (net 1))
 (arc (start 183.44 111.56) (mid 183.83598 111.72402) (end 184 112.12) (width 1) (layer "F.Cu") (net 1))
 (arc (start 183.44 69.56) (mid 183.83598 69.72402) (end 184 70.12) (width 1) (layer "F.Cu") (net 1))
 (arc (start 183.44 75.16) (mid 183.83598 75.32402) (end 184 75.72) (width 1) (layer "F.Cu") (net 1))
 (arc (start 183.44 136.76) (mid 183.83598 136.92402) (end 184 137.32) (width 1) (layer "F.Cu") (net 1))
 (arc (start 79 136.2) (mid 79.16402 136.59598) (end 79.56 136.76) (width 1) (layer "F.Cu") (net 1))
 (arc (start 183.44 55.56) (mid 183.83598 55.72402) (end 184 56.12) (width 1) (layer "F.Cu") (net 1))
 (arc (start 79 133.4) (mid 79.16402 133.79598) (end 79.56 133.96) (width 1) (layer "F.Cu") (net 1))
 (arc (start 79.56 110.16) (mid 79.16402 110.32402) (end 79 110.72) (width 1) (layer "F.Cu") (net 1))
 (arc (start 184 70.4) (mid 183.83598 70.79598) (end 183.44 70.96) (width 1) (layer "F.Cu") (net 1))
 (arc (start 184 73.2) (mid 183.83598 73.59598) (end 183.44 73.76) (width 1) (layer "F.Cu") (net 1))
 (arc (start 184 109.6) (mid 183.83598 109.99598) (end 183.44 110.16) (width 1) (layer "F.Cu") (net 1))
 (arc (start 79.56 138.16) (mid 79.16402 138.32402) (end 79 138.72) (width 1) (layer "F.Cu") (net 1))
 (arc (start 79.56 87.76) (mid 79.16402 87.92402) (end 79 88.32) (width 1) (layer "F.Cu") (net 1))
 (arc (start 79.56 118.56) (mid 79.16402 118.72402) (end 79 119.12) (width 1) (layer "F.Cu") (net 1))
 (arc (start 184 126.4) (mid 183.83598 126.79598) (end 183.44 126.96) (width 1) (layer "F.Cu") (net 1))
 (arc (start 184 84.4) (mid 183.83598 84.79598) (end 183.44 84.96) (width 1) (layer "F.Cu") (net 1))
 (arc (start 183.44 44.36) (mid 183.83598 44.52402) (end 184 44.92) (width 1) (layer "F.Cu") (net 1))
 (arc (start 184 56.4) (mid 183.83598 56.79598) (end 183.44 56.96) (width 1) (layer "F.Cu") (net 1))
 (arc (start 79.56 115.76) (mid 79.16402 115.92402) (end 79 116.32) (width 1) (layer "F.Cu") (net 1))
 (arc (start 183.44 133.96) (mid 183.83598 134.12402) (end 184 134.52) (width 1) (layer "F.Cu") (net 1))
 (arc (start 184 118) (mid 183.83598 118.39598) (end 183.44 118.56) (width 1) (layer "F.Cu") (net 1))
 (arc (start 79 99.8) (mid 79.16402 100.19598) (end 79.56 100.36) (width 1) (layer "F.Cu") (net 1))
 (arc (start 79.56 112.96) (mid 79.16402 113.12402) (end 79 113.52) (width 1) (layer "F.Cu") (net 1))
 (arc (start 184 34) (mid 183.83598 34.39598) (end 183.44 34.56) (width 1) (layer "F.Cu") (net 1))
 (arc (start 184 104) (mid 183.83598 104.39598) (end 183.44 104.56) (width 1) (layer "F.Cu") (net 1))
 (arc (start 79 69) (mid 79.16402 69.39598) (end 79.56 69.56) (width 1) (layer "F.Cu") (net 1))
 (arc (start 79 41) (mid 79.16402 41.39598) (end 79.56 41.56) (width 1) (layer "F.Cu") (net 1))
 (arc (start 79.56 45.76) (mid 79.16402 45.92402) (end 79 46.32) (width 1) (layer "F.Cu") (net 1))
 (arc (start 184 81.6) (mid 183.83598 81.99598) (end 183.44 82.16) (width 1) (layer "F.Cu") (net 1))
 (arc (start 79 111) (mid 79.16402 111.39598) (end 79.56 111.56) (width 1) (layer "F.Cu") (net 1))
 (arc (start 183.44 89.16) (mid 183.83598 89.32402) (end 184 89.72) (width 1) (layer "F.Cu") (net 1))
 (arc (start 184 45.2) (mid 183.83598 45.59598) (end 183.44 45.76) (width 1) (layer "F.Cu") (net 1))
 (arc (start 79.56 56.96) (mid 79.16402 57.12402) (end 79 57.52) (width 1) (layer "F.Cu") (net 1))
 (arc (start 184 101.2) (mid 183.83598 101.59598) (end 183.44 101.76) (width 1) (layer "F.Cu") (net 1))
 (arc (start 183.44 122.76) (mid 183.83598 122.92402) (end 184 123.32) (width 1) (layer "F.Cu") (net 1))
 (arc (start 79.56 42.96) (mid 79.16402 43.12402) (end 79 43.52) (width 1) (layer "F.Cu") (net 1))
 (arc (start 183.44 119.96) (mid 183.83598 120.12402) (end 184 120.52) (width 1) (layer "F.Cu") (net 1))
 (arc (start 79.56 76.56) (mid 79.16402 76.72402) (end 79 77.12) (width 1) (layer "F.Cu") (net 1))
 (arc (start 79 97) (mid 79.16402 97.39598) (end 79.56 97.56) (width 1) (layer "F.Cu") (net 1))
 (arc (start 79.56 34.56) (mid 79.16402 34.72402) (end 79 35.12) (width 1) (layer "F.Cu") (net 1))
 (arc (start 79.56 84.96) (mid 79.16402 85.12402) (end 79 85.52) (width 1) (layer "F.Cu") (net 1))
 (arc (start 79.56 65.36) (mid 79.16402 65.52402) (end 79 65.92) (width 1) (layer "F.Cu") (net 1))
 (arc (start 183.44 77.96) (mid 183.83598 78.12402) (end 184 78.52) (width 1) (layer "F.Cu") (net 1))
 (arc (start 79 130.6) (mid 79.16402 130.99598) (end 79.56 131.16) (width 1) (layer "F.Cu") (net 1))
 (arc (start 183.44 100.36) (mid 183.83598 100.52402) (end 184 100.92) (width 1) (layer "F.Cu") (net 1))
 (arc (start 79.56 40.16) (mid 79.16402 40.32402) (end 79 40.72) (width 1) (layer "F.Cu") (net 1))
 (arc (start 79 55) (mid 79.16402 55.39598) (end 79.56 55.56) (width 1) (layer "F.Cu") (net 1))
 (arc (start 184 92.8) (mid 183.83598 93.19598) (end 183.44 93.36) (width 1) (layer "F.Cu") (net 1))
 (arc (start 183.44 47.16) (mid 183.83598 47.32402) (end 184 47.72) (width 1) (layer "F.Cu") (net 1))
 (arc (start 79 35.4) (mid 79.16402 35.79598) (end 79.56 35.96) (width 1) (layer "F.Cu") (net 1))
 (arc (start 79 108.2) (mid 79.16402 108.59598) (end 79.56 108.76) (width 1) (layer "F.Cu") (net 1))
 (arc (start 79 91.4) (mid 79.16402 91.79598) (end 79.56 91.96) (width 1) (layer "F.Cu") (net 1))
 (arc (start 184 132) (mid 183.83598 132.39598) (end 183.44 132.56) (width 1) (layer "F.Cu") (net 1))
 (arc (start 79 80.2) (mid 79.16402 80.59598) (end 79.56 80.76) (width 1) (layer "F.Cu") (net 1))
 (arc (start 183.44 83.56) (mid 183.83598 83.72402) (end 184 84.12) (width 1) (layer "F.Cu") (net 1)))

